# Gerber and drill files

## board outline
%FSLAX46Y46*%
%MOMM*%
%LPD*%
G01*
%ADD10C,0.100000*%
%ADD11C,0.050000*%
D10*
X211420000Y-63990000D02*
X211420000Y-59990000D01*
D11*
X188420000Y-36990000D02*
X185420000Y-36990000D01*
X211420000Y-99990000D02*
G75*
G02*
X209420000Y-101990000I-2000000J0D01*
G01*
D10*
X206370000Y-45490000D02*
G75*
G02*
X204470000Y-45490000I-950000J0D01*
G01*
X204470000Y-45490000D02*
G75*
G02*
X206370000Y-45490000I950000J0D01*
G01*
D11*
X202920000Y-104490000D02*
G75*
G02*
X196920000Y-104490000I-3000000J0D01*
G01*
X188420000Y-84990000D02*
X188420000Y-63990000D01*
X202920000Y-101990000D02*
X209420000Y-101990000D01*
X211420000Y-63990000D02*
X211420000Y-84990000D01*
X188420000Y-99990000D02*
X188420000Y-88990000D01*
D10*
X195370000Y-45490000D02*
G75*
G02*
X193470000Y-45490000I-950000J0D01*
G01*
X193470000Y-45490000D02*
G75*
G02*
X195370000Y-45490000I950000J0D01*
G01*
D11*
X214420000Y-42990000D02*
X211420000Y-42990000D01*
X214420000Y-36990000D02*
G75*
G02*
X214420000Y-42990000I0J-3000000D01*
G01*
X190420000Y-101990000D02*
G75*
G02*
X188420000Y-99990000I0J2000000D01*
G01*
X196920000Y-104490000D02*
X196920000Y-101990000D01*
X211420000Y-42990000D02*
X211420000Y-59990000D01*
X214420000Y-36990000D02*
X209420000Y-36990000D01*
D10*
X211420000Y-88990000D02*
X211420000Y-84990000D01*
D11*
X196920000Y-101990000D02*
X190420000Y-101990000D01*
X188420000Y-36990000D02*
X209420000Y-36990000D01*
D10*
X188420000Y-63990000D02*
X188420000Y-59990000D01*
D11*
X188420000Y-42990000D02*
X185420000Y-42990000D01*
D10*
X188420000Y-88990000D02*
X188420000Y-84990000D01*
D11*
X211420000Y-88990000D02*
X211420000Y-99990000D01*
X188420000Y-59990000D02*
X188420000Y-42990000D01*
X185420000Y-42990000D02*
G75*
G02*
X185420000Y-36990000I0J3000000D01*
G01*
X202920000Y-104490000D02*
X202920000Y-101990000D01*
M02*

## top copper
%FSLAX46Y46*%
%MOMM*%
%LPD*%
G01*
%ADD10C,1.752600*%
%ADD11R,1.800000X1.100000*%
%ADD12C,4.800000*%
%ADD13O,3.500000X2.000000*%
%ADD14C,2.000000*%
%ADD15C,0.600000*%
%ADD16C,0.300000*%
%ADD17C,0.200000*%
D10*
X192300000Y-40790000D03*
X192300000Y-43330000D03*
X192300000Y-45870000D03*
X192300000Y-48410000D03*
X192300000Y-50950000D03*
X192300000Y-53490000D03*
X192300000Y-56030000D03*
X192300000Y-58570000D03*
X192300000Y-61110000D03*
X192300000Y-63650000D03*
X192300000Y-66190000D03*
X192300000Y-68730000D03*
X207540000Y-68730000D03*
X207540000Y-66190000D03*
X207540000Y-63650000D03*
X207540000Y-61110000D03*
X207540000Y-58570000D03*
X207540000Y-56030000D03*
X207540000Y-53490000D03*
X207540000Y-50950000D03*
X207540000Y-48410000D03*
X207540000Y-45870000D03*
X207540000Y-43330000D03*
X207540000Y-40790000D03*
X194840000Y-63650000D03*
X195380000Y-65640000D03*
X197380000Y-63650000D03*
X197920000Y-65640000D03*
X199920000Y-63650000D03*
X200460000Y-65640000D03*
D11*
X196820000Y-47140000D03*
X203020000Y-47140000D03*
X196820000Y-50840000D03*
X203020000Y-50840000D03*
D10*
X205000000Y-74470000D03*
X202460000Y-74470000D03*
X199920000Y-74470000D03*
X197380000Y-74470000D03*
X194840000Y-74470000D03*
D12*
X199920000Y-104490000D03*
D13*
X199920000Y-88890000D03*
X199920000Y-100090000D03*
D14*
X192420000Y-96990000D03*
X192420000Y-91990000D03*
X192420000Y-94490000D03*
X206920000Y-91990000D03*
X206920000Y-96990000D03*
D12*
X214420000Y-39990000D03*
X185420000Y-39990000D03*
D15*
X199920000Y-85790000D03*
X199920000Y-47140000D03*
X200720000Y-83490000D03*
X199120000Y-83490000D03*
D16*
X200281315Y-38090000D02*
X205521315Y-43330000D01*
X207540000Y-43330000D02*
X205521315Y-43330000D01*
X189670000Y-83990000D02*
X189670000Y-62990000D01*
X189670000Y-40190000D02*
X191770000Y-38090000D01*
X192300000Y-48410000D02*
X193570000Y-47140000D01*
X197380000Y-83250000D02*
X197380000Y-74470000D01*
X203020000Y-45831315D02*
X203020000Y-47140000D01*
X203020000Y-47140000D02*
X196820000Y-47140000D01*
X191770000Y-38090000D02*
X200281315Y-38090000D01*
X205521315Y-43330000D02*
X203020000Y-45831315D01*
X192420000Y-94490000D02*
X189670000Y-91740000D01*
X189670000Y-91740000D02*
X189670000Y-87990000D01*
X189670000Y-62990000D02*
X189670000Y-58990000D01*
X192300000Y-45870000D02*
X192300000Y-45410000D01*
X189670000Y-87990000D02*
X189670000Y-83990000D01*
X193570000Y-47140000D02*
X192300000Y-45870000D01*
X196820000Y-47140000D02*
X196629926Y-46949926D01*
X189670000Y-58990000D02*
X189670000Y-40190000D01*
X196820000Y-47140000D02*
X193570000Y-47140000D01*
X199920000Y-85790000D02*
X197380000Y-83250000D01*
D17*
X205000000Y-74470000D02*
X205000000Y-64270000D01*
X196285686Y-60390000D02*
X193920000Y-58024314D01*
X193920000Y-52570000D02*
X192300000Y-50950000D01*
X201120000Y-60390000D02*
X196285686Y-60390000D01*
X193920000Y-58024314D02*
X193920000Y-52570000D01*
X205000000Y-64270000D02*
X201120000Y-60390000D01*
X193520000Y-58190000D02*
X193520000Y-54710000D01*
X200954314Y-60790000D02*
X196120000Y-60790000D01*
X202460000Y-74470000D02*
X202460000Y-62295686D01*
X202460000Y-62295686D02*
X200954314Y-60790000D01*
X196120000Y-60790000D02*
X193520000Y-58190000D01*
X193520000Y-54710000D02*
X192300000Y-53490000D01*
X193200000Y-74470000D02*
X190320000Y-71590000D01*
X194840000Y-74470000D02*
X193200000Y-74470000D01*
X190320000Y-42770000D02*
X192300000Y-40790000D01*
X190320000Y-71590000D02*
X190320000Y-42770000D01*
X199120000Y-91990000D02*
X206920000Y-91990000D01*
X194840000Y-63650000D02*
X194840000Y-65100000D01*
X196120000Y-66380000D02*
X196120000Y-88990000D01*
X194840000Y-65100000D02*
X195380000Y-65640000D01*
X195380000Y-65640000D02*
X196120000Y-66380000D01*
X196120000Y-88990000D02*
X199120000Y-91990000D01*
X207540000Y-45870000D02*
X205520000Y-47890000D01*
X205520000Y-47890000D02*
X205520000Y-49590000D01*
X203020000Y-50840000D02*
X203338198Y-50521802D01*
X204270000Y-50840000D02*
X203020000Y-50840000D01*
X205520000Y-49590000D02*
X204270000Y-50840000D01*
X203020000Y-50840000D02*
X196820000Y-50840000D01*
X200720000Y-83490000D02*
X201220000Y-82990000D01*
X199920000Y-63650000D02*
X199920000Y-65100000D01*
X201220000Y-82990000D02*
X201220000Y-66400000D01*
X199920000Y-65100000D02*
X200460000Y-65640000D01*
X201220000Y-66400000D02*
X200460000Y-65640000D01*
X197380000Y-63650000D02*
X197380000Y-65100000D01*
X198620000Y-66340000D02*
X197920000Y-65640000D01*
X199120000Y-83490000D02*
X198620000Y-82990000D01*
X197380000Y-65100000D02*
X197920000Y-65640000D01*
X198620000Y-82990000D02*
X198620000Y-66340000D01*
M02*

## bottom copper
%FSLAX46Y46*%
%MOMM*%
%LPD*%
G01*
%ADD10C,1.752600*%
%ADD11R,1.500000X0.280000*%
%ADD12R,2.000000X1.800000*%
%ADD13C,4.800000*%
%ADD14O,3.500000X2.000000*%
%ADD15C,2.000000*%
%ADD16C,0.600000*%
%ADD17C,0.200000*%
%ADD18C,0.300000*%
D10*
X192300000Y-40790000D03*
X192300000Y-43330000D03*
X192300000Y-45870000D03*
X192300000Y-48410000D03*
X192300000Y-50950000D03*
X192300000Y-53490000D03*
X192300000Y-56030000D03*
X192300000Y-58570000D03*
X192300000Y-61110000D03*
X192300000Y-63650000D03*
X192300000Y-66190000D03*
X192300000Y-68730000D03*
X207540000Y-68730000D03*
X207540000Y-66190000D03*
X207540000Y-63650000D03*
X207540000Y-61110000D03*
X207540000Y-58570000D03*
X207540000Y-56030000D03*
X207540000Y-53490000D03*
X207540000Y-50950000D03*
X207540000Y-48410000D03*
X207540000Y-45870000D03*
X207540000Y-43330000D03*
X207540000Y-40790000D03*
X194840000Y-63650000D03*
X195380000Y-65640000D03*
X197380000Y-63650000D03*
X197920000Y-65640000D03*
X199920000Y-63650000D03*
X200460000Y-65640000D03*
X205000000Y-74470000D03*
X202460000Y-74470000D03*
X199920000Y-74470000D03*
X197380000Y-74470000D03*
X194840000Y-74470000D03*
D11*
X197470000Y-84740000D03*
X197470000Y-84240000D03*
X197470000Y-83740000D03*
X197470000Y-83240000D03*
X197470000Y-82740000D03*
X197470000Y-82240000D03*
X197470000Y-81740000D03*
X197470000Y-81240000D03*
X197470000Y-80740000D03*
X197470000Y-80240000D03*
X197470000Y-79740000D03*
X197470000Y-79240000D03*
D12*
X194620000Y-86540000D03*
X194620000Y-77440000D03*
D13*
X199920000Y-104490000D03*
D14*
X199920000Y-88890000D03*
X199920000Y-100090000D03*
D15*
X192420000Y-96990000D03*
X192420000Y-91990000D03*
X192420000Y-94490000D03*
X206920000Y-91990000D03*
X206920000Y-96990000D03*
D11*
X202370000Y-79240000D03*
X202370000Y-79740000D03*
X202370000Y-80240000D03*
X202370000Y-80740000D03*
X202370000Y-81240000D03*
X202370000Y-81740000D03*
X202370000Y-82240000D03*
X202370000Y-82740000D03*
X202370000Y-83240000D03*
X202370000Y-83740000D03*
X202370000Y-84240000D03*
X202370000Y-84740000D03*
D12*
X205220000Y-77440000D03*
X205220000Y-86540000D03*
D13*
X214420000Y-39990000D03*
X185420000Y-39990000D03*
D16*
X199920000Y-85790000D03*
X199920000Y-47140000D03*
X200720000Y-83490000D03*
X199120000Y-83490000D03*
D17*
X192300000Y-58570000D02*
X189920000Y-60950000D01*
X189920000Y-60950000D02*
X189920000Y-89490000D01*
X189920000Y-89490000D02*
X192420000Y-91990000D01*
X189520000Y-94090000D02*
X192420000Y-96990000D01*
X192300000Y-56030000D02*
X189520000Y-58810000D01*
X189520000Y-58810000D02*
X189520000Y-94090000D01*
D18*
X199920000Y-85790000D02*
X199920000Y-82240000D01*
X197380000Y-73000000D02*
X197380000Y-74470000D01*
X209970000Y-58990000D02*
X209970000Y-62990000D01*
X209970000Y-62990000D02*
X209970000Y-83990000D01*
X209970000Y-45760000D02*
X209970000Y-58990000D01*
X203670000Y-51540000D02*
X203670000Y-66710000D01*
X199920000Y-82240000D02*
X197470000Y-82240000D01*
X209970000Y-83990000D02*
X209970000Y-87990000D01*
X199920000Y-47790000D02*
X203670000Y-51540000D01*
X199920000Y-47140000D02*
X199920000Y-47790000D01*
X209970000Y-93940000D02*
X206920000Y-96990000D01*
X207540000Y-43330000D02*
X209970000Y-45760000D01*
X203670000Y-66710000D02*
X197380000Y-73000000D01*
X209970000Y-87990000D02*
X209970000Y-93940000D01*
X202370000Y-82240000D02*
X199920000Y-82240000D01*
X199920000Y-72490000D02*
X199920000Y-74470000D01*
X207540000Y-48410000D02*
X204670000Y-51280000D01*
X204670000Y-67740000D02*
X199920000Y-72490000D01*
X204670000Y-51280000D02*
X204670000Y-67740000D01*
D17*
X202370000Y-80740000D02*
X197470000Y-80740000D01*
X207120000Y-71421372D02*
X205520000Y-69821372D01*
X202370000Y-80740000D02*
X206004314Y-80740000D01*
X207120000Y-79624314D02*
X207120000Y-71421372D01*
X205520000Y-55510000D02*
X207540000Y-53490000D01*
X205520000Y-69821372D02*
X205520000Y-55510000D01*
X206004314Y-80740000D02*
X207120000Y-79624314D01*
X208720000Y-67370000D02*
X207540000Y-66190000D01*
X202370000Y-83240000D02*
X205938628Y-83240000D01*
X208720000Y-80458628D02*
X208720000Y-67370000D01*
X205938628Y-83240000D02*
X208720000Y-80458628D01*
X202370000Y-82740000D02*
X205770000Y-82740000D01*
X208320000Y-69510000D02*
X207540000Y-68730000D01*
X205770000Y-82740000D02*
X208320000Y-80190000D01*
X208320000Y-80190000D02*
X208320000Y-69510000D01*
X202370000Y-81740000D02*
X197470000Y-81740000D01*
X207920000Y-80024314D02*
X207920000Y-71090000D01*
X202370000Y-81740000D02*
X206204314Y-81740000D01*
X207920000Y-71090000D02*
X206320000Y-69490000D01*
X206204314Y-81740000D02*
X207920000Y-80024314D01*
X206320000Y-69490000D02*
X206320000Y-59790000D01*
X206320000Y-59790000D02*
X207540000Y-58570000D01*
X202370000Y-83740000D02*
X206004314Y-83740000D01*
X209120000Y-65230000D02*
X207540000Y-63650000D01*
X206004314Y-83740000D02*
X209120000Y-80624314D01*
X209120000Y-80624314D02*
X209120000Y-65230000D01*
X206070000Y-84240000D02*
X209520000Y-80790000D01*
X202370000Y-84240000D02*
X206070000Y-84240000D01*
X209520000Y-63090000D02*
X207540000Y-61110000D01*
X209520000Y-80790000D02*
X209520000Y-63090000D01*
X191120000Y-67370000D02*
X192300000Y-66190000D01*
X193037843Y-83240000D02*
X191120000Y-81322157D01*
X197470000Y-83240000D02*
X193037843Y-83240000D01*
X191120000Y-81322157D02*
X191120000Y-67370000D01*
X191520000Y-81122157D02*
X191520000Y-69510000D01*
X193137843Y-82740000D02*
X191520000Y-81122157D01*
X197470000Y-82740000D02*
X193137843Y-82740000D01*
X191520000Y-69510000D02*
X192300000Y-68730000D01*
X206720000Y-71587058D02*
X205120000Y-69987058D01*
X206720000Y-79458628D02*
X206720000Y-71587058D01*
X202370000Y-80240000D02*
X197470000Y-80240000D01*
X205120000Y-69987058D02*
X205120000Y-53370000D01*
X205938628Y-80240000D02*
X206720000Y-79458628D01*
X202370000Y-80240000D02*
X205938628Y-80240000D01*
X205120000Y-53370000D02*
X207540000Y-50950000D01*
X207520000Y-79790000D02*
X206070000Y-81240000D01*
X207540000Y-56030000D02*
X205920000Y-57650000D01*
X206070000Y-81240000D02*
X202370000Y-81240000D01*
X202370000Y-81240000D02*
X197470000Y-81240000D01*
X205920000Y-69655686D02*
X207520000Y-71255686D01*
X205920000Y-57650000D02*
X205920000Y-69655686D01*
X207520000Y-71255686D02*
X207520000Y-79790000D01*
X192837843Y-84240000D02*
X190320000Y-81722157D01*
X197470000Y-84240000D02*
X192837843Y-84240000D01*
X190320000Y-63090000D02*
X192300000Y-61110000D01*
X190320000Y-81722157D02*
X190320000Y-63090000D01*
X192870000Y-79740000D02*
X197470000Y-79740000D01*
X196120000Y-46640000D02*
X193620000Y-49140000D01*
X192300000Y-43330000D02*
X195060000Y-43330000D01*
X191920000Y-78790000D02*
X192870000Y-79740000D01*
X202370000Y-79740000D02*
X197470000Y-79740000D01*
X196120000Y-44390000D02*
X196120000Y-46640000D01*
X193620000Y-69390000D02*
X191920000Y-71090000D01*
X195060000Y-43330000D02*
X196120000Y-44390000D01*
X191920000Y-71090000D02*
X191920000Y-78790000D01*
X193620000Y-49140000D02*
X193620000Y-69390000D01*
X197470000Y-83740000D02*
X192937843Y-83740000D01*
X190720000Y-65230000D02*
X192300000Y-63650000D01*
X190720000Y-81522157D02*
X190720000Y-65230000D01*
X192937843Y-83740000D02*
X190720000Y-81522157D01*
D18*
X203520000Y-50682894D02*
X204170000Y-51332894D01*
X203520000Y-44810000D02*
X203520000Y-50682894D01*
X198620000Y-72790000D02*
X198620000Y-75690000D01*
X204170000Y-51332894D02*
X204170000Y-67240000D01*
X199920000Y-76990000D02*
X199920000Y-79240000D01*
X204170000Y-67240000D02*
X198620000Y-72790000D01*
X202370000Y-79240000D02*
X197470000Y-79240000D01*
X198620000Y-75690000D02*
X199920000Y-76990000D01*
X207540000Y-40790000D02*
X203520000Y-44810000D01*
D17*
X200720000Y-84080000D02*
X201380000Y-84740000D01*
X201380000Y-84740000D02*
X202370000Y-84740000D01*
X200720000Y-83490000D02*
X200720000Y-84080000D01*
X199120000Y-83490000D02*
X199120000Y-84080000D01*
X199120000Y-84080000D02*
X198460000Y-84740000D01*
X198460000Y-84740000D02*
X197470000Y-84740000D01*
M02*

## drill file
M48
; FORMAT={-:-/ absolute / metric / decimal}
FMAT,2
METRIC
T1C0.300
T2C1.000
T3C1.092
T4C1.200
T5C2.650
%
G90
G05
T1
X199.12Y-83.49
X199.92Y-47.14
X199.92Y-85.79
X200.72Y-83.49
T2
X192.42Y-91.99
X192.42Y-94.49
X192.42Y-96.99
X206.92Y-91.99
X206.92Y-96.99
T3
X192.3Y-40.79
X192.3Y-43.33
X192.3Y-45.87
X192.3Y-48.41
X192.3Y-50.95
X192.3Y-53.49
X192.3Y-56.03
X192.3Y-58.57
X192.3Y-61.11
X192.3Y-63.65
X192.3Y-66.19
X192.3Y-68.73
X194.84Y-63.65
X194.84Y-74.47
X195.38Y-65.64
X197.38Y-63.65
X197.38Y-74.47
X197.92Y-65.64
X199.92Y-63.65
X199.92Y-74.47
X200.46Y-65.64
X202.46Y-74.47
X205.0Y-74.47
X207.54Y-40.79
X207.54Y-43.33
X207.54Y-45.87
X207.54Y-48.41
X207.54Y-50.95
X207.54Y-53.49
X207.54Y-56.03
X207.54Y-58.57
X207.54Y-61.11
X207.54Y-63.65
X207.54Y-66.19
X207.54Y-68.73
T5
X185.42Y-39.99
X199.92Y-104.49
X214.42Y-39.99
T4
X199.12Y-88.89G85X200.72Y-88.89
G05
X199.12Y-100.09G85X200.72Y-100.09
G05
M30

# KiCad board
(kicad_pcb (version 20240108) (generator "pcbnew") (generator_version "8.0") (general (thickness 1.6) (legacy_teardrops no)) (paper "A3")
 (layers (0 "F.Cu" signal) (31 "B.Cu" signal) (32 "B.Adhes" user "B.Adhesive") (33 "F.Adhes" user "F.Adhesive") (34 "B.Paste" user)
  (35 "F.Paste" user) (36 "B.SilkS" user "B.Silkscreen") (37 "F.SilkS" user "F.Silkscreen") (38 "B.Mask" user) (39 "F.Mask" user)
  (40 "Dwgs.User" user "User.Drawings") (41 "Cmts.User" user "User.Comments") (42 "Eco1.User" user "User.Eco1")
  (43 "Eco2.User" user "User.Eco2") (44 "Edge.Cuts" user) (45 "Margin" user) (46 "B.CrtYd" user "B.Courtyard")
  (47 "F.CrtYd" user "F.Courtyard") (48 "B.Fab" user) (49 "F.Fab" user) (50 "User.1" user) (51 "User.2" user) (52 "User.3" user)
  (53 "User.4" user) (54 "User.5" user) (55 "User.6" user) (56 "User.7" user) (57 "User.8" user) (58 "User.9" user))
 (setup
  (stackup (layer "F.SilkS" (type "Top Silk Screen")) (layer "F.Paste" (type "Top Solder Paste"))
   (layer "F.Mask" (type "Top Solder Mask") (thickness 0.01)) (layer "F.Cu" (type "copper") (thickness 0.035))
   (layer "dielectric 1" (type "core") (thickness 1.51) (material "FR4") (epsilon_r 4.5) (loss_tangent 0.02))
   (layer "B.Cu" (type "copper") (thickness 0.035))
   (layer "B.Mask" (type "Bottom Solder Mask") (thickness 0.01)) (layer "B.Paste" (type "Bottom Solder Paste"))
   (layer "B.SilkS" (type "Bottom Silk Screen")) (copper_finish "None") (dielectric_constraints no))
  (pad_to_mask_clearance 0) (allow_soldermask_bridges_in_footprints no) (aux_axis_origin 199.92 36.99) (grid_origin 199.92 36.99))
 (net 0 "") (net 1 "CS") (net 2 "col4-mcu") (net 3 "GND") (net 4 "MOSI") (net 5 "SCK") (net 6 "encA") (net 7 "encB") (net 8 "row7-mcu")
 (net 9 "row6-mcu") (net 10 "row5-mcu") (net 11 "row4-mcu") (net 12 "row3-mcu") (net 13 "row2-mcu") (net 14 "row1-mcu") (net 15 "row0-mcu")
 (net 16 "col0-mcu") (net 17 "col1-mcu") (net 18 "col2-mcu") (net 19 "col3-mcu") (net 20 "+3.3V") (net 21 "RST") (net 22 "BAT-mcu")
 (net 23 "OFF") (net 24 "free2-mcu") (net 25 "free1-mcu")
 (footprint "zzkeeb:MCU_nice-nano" (layer "F.Cu") (at 199.92 53.49)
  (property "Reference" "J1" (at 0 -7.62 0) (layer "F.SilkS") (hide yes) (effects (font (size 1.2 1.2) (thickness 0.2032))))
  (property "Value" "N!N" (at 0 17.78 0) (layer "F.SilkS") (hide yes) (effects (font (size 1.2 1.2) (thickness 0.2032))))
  (pad "1" thru_hole circle (at -7.62 -12.7 270) (size 1.7526 1.7526) (drill 1.0922) (layers "*.Cu" "*.Mask") (remove_unused_layers no)
   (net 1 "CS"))
  (pad "2" thru_hole circle (at -7.62 -10.16 270) (size 1.7526 1.7526) (drill 1.0922) (layers "*.Cu" "*.Mask") (remove_unused_layers no)
   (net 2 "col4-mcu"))
  (pad "3" thru_hole circle (at -7.62 -7.62 270) (size 1.7526 1.7526) (drill 1.0922) (layers "*.Cu" "*.Mask") (remove_unused_layers no)
   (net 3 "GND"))
  (pad "4" thru_hole circle (at -7.62 -5.08 270) (size 1.7526 1.7526) (drill 1.0922) (layers "*.Cu" "*.Mask") (remove_unused_layers no)
   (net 3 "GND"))
  (pad "5" thru_hole circle (at -7.62 -2.54 270) (size 1.7526 1.7526) (drill 1.0922) (layers "*.Cu" "*.Mask") (remove_unused_layers no)
   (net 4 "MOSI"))
  (pad "6" thru_hole circle (at -7.62 0 270) (size 1.7526 1.7526) (drill 1.0922) (layers "*.Cu" "*.Mask") (remove_unused_layers no)
   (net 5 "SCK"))
  (pad "7" thru_hole circle (at -7.62 2.54 270) (size 1.7526 1.7526) (drill 1.0922) (layers "*.Cu" "*.Mask") (remove_unused_layers no)
   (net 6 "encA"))
  (pad "8" thru_hole circle (at -7.62 5.08 270) (size 1.7526 1.7526) (drill 1.0922) (layers "*.Cu" "*.Mask") (remove_unused_layers no)
   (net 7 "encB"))
  (pad "9" thru_hole circle (at -7.62 7.62 270) (size 1.7526 1.7526) (drill 1.0922) (layers "*.Cu" "*.Mask") (remove_unused_layers no)
   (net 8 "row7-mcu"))
  (pad "10" thru_hole circle (at -7.62 10.16 270) (size 1.7526 1.7526) (drill 1.0922) (layers "*.Cu" "*.Mask") (remove_unused_layers no)
   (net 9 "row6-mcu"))
  (pad "11" thru_hole circle (at -7.62 12.7 270) (size 1.7526 1.7526) (drill 1.0922) (layers "*.Cu" "*.Mask") (remove_unused_layers no)
   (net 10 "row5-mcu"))
  (pad "12" thru_hole circle (at -7.62 15.24 270) (size 1.7526 1.7526) (drill 1.0922) (layers "*.Cu" "*.Mask") (remove_unused_layers no)
   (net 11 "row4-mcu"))
  (pad "13" thru_hole circle (at 7.62 15.24 270) (size 1.7526 1.7526) (drill 1.0922) (layers "*.Cu" "*.Mask") (remove_unused_layers no)
   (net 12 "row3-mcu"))
  (pad "14" thru_hole circle (at 7.62 12.7 270) (size 1.7526 1.7526) (drill 1.0922) (layers "*.Cu" "*.Mask") (remove_unused_layers no)
   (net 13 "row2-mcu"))
  (pad "15" thru_hole circle (at 7.62 10.16 270) (size 1.7526 1.7526) (drill 1.0922) (layers "*.Cu" "*.Mask") (remove_unused_layers no)
   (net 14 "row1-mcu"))
  (pad "16" thru_hole circle (at 7.62 7.62 270) (size 1.7526 1.7526) (drill 1.0922) (layers "*.Cu" "*.Mask") (remove_unused_layers no)
   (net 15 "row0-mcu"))
  (pad "17" thru_hole circle (at 7.62 5.08 270) (size 1.7526 1.7526) (drill 1.0922) (layers "*.Cu" "*.Mask") (remove_unused_layers no)
   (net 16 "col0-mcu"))
  (pad "18" thru_hole circle (at 7.62 2.54 270) (size 1.7526 1.7526) (drill 1.0922) (layers "*.Cu" "*.Mask") (remove_unused_layers no)
   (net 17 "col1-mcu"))
  (pad "19" thru_hole circle (at 7.62 0 270) (size 1.7526 1.7526) (drill 1.0922) (layers "*.Cu" "*.Mask") (remove_unused_layers no)
   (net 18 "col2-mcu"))
  (pad "20" thru_hole circle (at 7.62 -2.54 270) (size 1.7526 1.7526) (drill 1.0922) (layers "*.Cu" "*.Mask") (remove_unused_layers no)
   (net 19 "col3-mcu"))
  (pad "21" thru_hole circle (at 7.62 -5.08 270) (size 1.7526 1.7526) (drill 1.0922) (layers "*.Cu" "*.Mask") (remove_unused_layers no)
   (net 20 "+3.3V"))
  (pad "22" thru_hole circle (at 7.62 -7.62 270) (size 1.7526 1.7526) (drill 1.0922) (layers "*.Cu" "*.Mask") (remove_unused_layers no)
   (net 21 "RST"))
  (pad "23" thru_hole circle (at 7.62 -10.16 270) (size 1.7526 1.7526) (drill 1.0922) (layers "*.Cu" "*.Mask") (remove_unused_layers no)
   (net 3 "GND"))
  (pad "24" thru_hole circle (at 7.62 -12.7 270) (size 1.7526 1.7526) (drill 1.0922) (layers "*.Cu" "*.Mask") (remove_unused_layers no)
   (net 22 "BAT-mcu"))
  (pad "31" thru_hole circle (at -5.08 10.16 270) (size 1.7526 1.7526) (drill 1.0922) (layers "*.Cu" "*.Mask") (remove_unused_layers no)
   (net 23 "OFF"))
  (pad "31" thru_hole circle (at -4.54 12.15 270) (size 1.7526 1.7526) (drill 1.0922) (layers "*.Cu" "*.Mask") (remove_unused_layers no)
   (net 23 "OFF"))
  (pad "32" thru_hole circle (at -2.54 10.16 270) (size 1.7526 1.7526) (drill 1.0922) (layers "*.Cu" "*.Mask") (remove_unused_layers no)
   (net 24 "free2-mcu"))
  (pad "32" thru_hole circle (at -2 12.15 270) (size 1.7526 1.7526) (drill 1.0922) (layers "*.Cu" "*.Mask") (remove_unused_layers no)
   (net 24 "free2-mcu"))
  (pad "33" thru_hole circle (at 0 10.16 270) (size 1.7526 1.7526) (drill 1.0922) (layers "*.Cu" "*.Mask") (remove_unused_layers no)
   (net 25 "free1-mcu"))
  (pad "33" thru_hole circle (at 0.54 12.15 270) (size 1.7526 1.7526) (drill 1.0922) (layers "*.Cu" "*.Mask") (remove_unused_layers no)
   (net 25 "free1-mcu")))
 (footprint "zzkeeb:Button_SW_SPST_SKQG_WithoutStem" (layer "F.Cu") (at 199.92 48.99)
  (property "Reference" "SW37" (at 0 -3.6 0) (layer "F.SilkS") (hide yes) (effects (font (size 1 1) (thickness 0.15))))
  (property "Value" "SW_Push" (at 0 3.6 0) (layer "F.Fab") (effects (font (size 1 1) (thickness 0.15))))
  (pad "1" smd rect (at -3.1 -1.85) (size 1.8 1.1) (layers "F.Cu" "F.Paste" "F.Mask") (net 3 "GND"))
  (pad "1" smd rect (at 3.1 -1.85) (size 1.8 1.1) (layers "F.Cu" "F.Paste" "F.Mask") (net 3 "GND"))
  (pad "2" smd rect (at -3.1 1.85) (size 1.8 1.1) (layers "F.Cu" "F.Paste" "F.Mask") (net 21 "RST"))
  (pad "2" smd rect (at 3.1 1.85) (size 1.8 1.1) (layers "F.Cu" "F.Paste" "F.Mask") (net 21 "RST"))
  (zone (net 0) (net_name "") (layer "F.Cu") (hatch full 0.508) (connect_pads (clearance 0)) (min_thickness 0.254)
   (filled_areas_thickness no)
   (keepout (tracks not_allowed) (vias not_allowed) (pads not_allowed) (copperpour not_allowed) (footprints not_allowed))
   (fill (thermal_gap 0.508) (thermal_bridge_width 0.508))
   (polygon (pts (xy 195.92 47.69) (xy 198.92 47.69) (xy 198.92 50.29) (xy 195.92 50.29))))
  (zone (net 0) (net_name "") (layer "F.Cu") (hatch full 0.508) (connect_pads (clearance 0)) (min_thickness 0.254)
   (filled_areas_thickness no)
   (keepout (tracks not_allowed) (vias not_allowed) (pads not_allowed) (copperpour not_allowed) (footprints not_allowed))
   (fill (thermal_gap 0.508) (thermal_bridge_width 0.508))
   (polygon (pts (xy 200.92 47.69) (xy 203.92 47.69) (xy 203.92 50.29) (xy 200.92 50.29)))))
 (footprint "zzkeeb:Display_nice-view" (layer "B.Cu") (at 199.92 57.99 180)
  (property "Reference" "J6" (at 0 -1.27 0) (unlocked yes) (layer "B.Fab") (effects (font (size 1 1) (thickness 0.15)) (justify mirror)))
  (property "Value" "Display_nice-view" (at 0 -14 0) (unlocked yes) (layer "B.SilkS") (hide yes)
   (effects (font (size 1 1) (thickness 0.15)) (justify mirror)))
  (pad "1" thru_hole circle (at -5.08 -16.48 180) (size 1.7526 1.7526) (drill 1.0922) (layers "*.Cu" "*.Mask") (remove_unused_layers no)
   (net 4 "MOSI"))
  (pad "2" thru_hole circle (at -2.54 -16.48 180) (size 1.7526 1.7526) (drill 1.0922) (layers "*.Cu" "*.Mask") (remove_unused_layers no)
   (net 5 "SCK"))
  (pad "3" thru_hole circle (at 0 -16.48 180) (size 1.7526 1.7526) (drill 1.0922) (layers "*.Cu" "*.Mask") (remove_unused_layers no)
   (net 20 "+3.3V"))
  (pad "4" thru_hole circle (at 2.54 -16.48 180) (size 1.7526 1.7526) (drill 1.0922) (layers "*.Cu" "*.Mask") (remove_unused_layers no)
   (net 3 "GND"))
  (pad "5" thru_hole circle (at 5.08 -16.48 180) (size 1.7526 1.7526) (drill 1.0922) (layers "*.Cu" "*.Mask") (remove_unused_layers no)
   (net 1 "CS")))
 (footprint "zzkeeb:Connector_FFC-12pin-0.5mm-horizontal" (layer "B.Cu") (at 195.92 81.99 90)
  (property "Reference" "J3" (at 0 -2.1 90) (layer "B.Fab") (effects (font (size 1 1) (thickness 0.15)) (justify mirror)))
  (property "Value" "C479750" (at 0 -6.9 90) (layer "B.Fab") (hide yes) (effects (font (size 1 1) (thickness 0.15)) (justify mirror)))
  (pad "1" smd rect (at -2.75 1.55 90) (size 0.28 1.5) (layers "B.Cu" "B.Paste" "B.Mask") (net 24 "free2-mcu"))
  (pad "2" smd rect (at -2.25 1.55 90) (size 0.28 1.5) (layers "B.Cu" "B.Paste" "B.Mask") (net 8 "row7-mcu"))
  (pad "3" smd rect (at -1.75 1.55 90) (size 0.28 1.5) (layers "B.Cu" "B.Paste" "B.Mask") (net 9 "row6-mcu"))
  (pad "4" smd rect (at -1.25 1.55 90) (size 0.28 1.5) (layers "B.Cu" "B.Paste" "B.Mask") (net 10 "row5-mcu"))
  (pad "5" smd rect (at -0.75 1.55 90) (size 0.28 1.5) (layers "B.Cu" "B.Paste" "B.Mask") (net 11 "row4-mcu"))
  (pad "6" smd rect (at -0.25 1.55 90) (size 0.28 1.5) (layers "B.Cu" "B.Paste" "B.Mask") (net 3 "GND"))
  (pad "7" smd rect (at 0.25 1.55 90) (size 0.28 1.5) (layers "B.Cu" "B.Paste" "B.Mask") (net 16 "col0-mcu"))
  (pad "8" smd rect (at 0.75 1.55 90) (size 0.28 1.5) (layers "B.Cu" "B.Paste" "B.Mask") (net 17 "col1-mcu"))
  (pad "9" smd rect (at 1.25 1.55 90) (size 0.28 1.5) (layers "B.Cu" "B.Paste" "B.Mask") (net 18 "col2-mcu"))
  (pad "10" smd rect (at 1.75 1.55 90) (size 0.28 1.5) (layers "B.Cu" "B.Paste" "B.Mask") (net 19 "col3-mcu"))
  (pad "11" smd rect (at 2.25 1.55 90) (size 0.28 1.5) (layers "B.Cu" "B.Paste" "B.Mask") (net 2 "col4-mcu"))
  (pad "12" smd rect (at 2.75 1.55 90) (size 0.28 1.5) (layers "B.Cu" "B.Paste" "B.Mask") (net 22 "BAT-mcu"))
  (pad "MP" smd rect (at -4.55 -1.3 90) (size 1.8 2) (layers "B.Cu" "B.Paste" "B.Mask"))
  (pad "MP" smd rect (at 4.55 -1.3 90) (size 1.8 2) (layers "B.Cu" "B.Paste" "B.Mask")))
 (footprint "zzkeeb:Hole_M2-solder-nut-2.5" (layer "B.Cu") (at 199.92 104.49 180)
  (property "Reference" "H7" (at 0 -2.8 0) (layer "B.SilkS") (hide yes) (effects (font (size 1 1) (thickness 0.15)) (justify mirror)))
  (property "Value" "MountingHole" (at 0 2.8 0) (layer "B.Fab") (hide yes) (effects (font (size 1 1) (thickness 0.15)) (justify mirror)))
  (pad "" thru_hole circle (at 0 0 180) (size 4.8 4.8) (drill 2.65) (layers "*.Cu" "B.Mask") (remove_unused_layers no)))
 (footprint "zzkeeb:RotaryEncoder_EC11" (layer "B.Cu") (at 199.92 94.49)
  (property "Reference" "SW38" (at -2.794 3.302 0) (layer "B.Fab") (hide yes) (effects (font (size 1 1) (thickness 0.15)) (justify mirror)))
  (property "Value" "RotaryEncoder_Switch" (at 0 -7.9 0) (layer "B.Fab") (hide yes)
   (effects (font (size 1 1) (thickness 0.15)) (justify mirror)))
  (pad "" thru_hole oval (at 0 -5.6) (size 3.5 2) (drill oval 2.8 1.2) (layers "*.Cu" "*.Mask") (remove_unused_layers no))
  (pad "" thru_hole oval (at 0 5.6) (size 3.5 2) (drill oval 2.8 1.2) (layers "*.Cu" "*.Mask") (remove_unused_layers no))
  (pad "A" thru_hole circle (at -7.5 2.5) (size 2 2) (drill 1) (layers "*.Cu" "F.Mask") (remove_unused_layers no) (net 6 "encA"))
  (pad "B" thru_hole circle (at -7.5 -2.5) (size 2 2) (drill 1) (layers "*.Cu" "F.Mask") (remove_unused_layers no) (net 7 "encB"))
  (pad "C" thru_hole circle (at -7.5 0) (size 2 2) (drill 1) (layers "*.Cu" "F.Mask") (remove_unused_layers no) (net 3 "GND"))
  (pad "S1" thru_hole circle (at 7 -2.5) (size 2 2) (drill 1) (layers "*.Cu" "F.Mask") (remove_unused_layers no) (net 23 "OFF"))
  (pad "S2" thru_hole circle (at 7 2.5) (size 2 2) (drill 1) (layers "*.Cu" "F.Mask") (remove_unused_layers no) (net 3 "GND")))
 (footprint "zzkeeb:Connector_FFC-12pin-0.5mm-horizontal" (layer "B.Cu") (at 203.92 81.99 -90)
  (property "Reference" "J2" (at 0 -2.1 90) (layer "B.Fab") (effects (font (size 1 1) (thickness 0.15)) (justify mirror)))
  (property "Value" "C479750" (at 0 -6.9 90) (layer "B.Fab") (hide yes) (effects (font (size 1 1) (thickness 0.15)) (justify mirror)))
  (pad "1" smd rect (at -2.75 1.55 270) (size 0.28 1.5) (layers "B.Cu" "B.Paste" "B.Mask") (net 22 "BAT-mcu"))
  (pad "2" smd rect (at -2.25 1.55 270) (size 0.28 1.5) (layers "B.Cu" "B.Paste" "B.Mask") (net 2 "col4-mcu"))
  (pad "3" smd rect (at -1.75 1.55 270) (size 0.28 1.5) (layers "B.Cu" "B.Paste" "B.Mask") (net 19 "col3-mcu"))
  (pad "4" smd rect (at -1.25 1.55 270) (size 0.28 1.5) (layers "B.Cu" "B.Paste" "B.Mask") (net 18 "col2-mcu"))
  (pad "5" smd rect (at -0.75 1.55 270) (size 0.28 1.5) (layers "B.Cu" "B.Paste" "B.Mask") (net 17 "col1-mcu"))
  (pad "6" smd rect (at -0.25 1.55 270) (size 0.28 1.5) (layers "B.Cu" "B.Paste" "B.Mask") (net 16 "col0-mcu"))
  (pad "7" smd rect (at 0.25 1.55 270) (size 0.28 1.5) (layers "B.Cu" "B.Paste" "B.Mask") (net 3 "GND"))
  (pad "8" smd rect (at 0.75 1.55 270) (size 0.28 1.5) (layers "B.Cu" "B.Paste" "B.Mask") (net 12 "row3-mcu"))
  (pad "9" smd rect (at 1.25 1.55 270) (size 0.28 1.5) (layers "B.Cu" "B.Paste" "B.Mask") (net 13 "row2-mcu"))
  (pad "10" smd rect (at 1.75 1.55 270) (size 0.28 1.5) (layers "B.Cu" "B.Paste" "B.Mask") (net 14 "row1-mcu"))
  (pad "11" smd rect (at 2.25 1.55 270) (size 0.28 1.5) (layers "B.Cu" "B.Paste" "B.Mask") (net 15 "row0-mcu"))
  (pad "12" smd rect (at 2.75 1.55 270) (size 0.28 1.5) (layers "B.Cu" "B.Paste" "B.Mask") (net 25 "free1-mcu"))
  (pad "MP" smd rect (at -4.55 -1.3 270) (size 1.8 2) (layers "B.Cu" "B.Paste" "B.Mask"))
  (pad "MP" smd rect (at 4.55 -1.3 270) (size 1.8 2) (layers "B.Cu" "B.Paste" "B.Mask")))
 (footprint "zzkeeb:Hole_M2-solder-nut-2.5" (layer "B.Cu") (at 214.42 39.99 180)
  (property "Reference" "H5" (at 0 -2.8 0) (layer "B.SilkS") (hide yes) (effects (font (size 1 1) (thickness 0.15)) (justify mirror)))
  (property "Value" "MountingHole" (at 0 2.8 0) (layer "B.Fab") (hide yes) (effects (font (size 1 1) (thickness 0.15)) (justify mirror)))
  (pad "" thru_hole circle (at 0 0 180) (size 4.8 4.8) (drill 2.65) (layers "*.Cu" "B.Mask") (remove_unused_layers no)))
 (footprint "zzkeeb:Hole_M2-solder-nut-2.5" (layer "B.Cu") (at 185.42 39.99 180)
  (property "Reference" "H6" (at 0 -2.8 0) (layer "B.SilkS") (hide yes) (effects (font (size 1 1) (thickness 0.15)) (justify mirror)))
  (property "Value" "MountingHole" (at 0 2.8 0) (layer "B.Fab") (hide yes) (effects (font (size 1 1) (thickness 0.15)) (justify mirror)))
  (pad "" thru_hole circle (at 0 0 180) (size 4.8 4.8) (drill 2.65) (layers "*.Cu" "B.Mask") (remove_unused_layers no)))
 (gr_line (start 211.42 63.99) (end 211.42 59.99) (stroke (width 0.1) (type default)) (layer "Edge.Cuts"))
 (gr_line (start 188.42 36.99) (end 185.42 36.99) (stroke (width 0.05) (type default)) (layer "Edge.Cuts"))
 (gr_arc (start 211.42 99.99) (mid 210.834213 101.404212) (end 209.42 101.99) (stroke (width 0.05) (type default)) (layer "Edge.Cuts"))
 (gr_circle (center 205.42 45.49) (end 206.37 45.49) (stroke (width 0.1) (type default)) (fill none) (layer "Edge.Cuts"))
 (gr_arc (start 202.92 104.49) (mid 199.92 107.49) (end 196.92 104.49) (stroke (width 0.05) (type default)) (layer "Edge.Cuts"))
 (gr_line (start 188.42 84.99) (end 188.42 63.99) (stroke (width 0.05) (type default)) (layer "Edge.Cuts"))
 (gr_line (start 202.92 101.99) (end 209.42 101.99) (stroke (width 0.05) (type default)) (layer "Edge.Cuts"))
 (gr_line (start 211.42 63.99) (end 211.42 84.99) (stroke (width 0.05) (type default)) (layer "Edge.Cuts"))
 (gr_line (start 188.42 99.99) (end 188.42 88.99) (stroke (width 0.05) (type default)) (layer "Edge.Cuts"))
 (gr_circle (center 194.42 45.49) (end 195.37 45.49) (stroke (width 0.1) (type default)) (fill none) (layer "Edge.Cuts"))
 (gr_line (start 214.42 42.99) (end 211.42 42.99) (stroke (width 0.05) (type default)) (layer "Edge.Cuts"))
 (gr_arc (start 214.42 36.99) (mid 217.42 39.99) (end 214.42 42.99) (stroke (width 0.05) (type default)) (layer "Edge.Cuts"))
 (gr_arc (start 190.42 101.99) (mid 189.005786 101.404214) (end 188.42 99.99) (stroke (width 0.05) (type default)) (layer "Edge.Cuts"))
 (gr_line (start 196.92 104.49) (end 196.92 101.99) (stroke (width 0.05) (type default)) (layer "Edge.Cuts"))
 (gr_line (start 211.42 42.99) (end 211.42 59.99) (stroke (width 0.05) (type default)) (layer "Edge.Cuts"))
 (gr_line (start 214.42 36.99) (end 209.42 36.99) (stroke (width 0.05) (type default)) (layer "Edge.Cuts"))
 (gr_line (start 211.42 88.99) (end 211.42 84.99) (stroke (width 0.1) (type default)) (layer "Edge.Cuts"))
 (gr_line (start 196.92 101.99) (end 190.42 101.99) (stroke (width 0.05) (type default)) (layer "Edge.Cuts"))
 (gr_line (start 188.42 36.99) (end 209.42 36.99) (stroke (width 0.05) (type default)) (layer "Edge.Cuts"))
 (gr_line (start 188.42 63.99) (end 188.42 59.99) (stroke (width 0.1) (type default)) (layer "Edge.Cuts"))
 (gr_line (start 188.42 42.99) (end 185.42 42.99) (stroke (width 0.05) (type default)) (layer "Edge.Cuts"))
 (gr_line (start 188.42 88.99) (end 188.42 84.99) (stroke (width 0.1) (type default)) (layer "Edge.Cuts"))
 (gr_line (start 211.42 88.99) (end 211.42 99.99) (stroke (width 0.05) (type default)) (layer "Edge.Cuts"))
 (gr_line (start 188.42 59.99) (end 188.42 42.99) (stroke (width 0.05) (type default)) (layer "Edge.Cuts"))
 (gr_arc (start 185.42 42.99) (mid 182.42 39.99) (end 185.42 36.99) (stroke (width 0.05) (type default)) (layer "Edge.Cuts"))
 (gr_line (start 202.92 104.49) (end 202.92 101.99) (stroke (width 0.05) (type default)) (layer "Edge.Cuts"))
 (segment (start 192.3 58.57) (end 189.92 60.95) (width 0.2) (layer "B.Cu") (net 7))
 (segment (start 189.92 60.95) (end 189.92 89.49) (width 0.2) (layer "B.Cu") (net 7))
 (segment (start 189.92 89.49) (end 192.42 91.99) (width 0.2) (layer "B.Cu") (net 7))
 (segment (start 189.52 94.09) (end 192.42 96.99) (width 0.2) (layer "B.Cu") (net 6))
 (segment (start 192.3 56.03) (end 189.52 58.81) (width 0.2) (layer "B.Cu") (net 6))
 (segment (start 189.52 58.81) (end 189.52 94.09) (width 0.2) (layer "B.Cu") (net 6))
 (segment (start 200.281315 38.09) (end 205.521315 43.33) (width 0.3) (layer "F.Cu") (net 3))
 (segment (start 207.54 43.33) (end 205.521315 43.33) (width 0.3) (layer "F.Cu") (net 3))
 (segment (start 189.67 83.99) (end 189.67 62.99) (width 0.3) (layer "F.Cu") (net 3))
 (segment (start 189.67 40.19) (end 191.77 38.09) (width 0.3) (layer "F.Cu") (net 3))
 (segment (start 192.3 48.41) (end 193.57 47.14) (width 0.3) (layer "F.Cu") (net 3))
 (segment (start 197.38 83.25) (end 197.38 74.47) (width 0.3) (layer "F.Cu") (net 3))
 (segment (start 203.02 45.831315) (end 203.02 47.14) (width 0.3) (layer "F.Cu") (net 3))
 (segment (start 203.02 47.14) (end 196.82 47.14) (width 0.3) (layer "F.Cu") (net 3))
 (segment (start 191.77 38.09) (end 200.281315 38.09) (width 0.3) (layer "F.Cu") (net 3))
 (segment (start 205.521315 43.33) (end 203.02 45.831315) (width 0.3) (layer "F.Cu") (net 3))
 (segment (start 192.42 94.49) (end 189.67 91.74) (width 0.3) (layer "F.Cu") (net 3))
 (segment (start 189.67 91.74) (end 189.67 87.99) (width 0.3) (layer "F.Cu") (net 3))
 (segment (start 189.67 62.99) (end 189.67 58.99) (width 0.3) (layer "F.Cu") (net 3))
 (segment (start 192.3 45.87) (end 192.3 45.41) (width 0.3) (layer "F.Cu") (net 3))
 (segment (start 189.67 87.99) (end 189.67 83.99) (width 0.3) (layer "F.Cu") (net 3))
 (segment (start 193.57 47.14) (end 192.3 45.87) (width 0.3) (layer "F.Cu") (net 3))
 (segment (start 196.82 47.14) (end 196.629926 46.949926) (width 0.3) (layer "F.Cu") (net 3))
 (segment (start 189.67 58.99) (end 189.67 40.19) (width 0.3) (layer "F.Cu") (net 3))
 (segment (start 196.82 47.14) (end 193.57 47.14) (width 0.3) (layer "F.Cu") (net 3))
 (segment (start 199.92 85.79) (end 197.38 83.25) (width 0.3) (layer "F.Cu") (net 3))
 (via (at 199.92 85.79) (size 0.6) (drill 0.3) (layers "F.Cu" "B.Cu") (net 3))
 (via (at 199.92 47.14) (size 0.6) (drill 0.3) (layers "F.Cu" "B.Cu") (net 3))
 (segment (start 199.92 85.79) (end 199.92 82.24) (width 0.3) (layer "B.Cu") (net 3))
 (segment (start 197.38 73) (end 197.38 74.47) (width 0.3) (layer "B.Cu") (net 3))
 (segment (start 209.97 58.99) (end 209.97 62.99) (width 0.3) (layer "B.Cu") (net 3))
 (segment (start 209.97 62.99) (end 209.97 83.99) (width 0.3) (layer "B.Cu") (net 3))
 (segment (start 209.97 45.76) (end 209.97 58.99) (width 0.3) (layer "B.Cu") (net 3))
 (segment (start 203.67 51.54) (end 203.67 66.71) (width 0.3) (layer "B.Cu") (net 3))
 (segment (start 199.92 82.24) (end 197.47 82.24) (width 0.3) (layer "B.Cu") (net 3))
 (segment (start 209.97 83.99) (end 209.97 87.99) (width 0.3) (layer "B.Cu") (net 3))
 (segment (start 199.92 47.79) (end 203.67 51.54) (width 0.3) (layer "B.Cu") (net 3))
 (segment (start 199.92 47.14) (end 199.92 47.79) (width 0.3) (layer "B.Cu") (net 3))
 (segment (start 209.97 93.94) (end 206.92 96.99) (width 0.3) (layer "B.Cu") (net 3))
 (segment (start 207.54 43.33) (end 209.97 45.76) (width 0.3) (layer "B.Cu") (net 3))
 (segment (start 203.67 66.71) (end 197.38 73) (width 0.3) (layer "B.Cu") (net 3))
 (segment (start 209.97 87.99) (end 209.97 93.94) (width 0.3) (layer "B.Cu") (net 3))
 (segment (start 202.37 82.24) (end 199.92 82.24) (width 0.3) (layer "B.Cu") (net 3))
 (segment (start 205 74.47) (end 205 64.27) (width 0.2) (layer "F.Cu") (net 4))
 (segment (start 196.285686 60.39) (end 193.92 58.024314) (width 0.2) (layer "F.Cu") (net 4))
 (segment (start 193.92 52.57) (end 192.3 50.95) (width 0.2) (layer "F.Cu") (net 4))
 (segment (start 201.12 60.39) (end 196.285686 60.39) (width 0.2) (layer "F.Cu") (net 4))
 (segment (start 193.92 58.024314) (end 193.92 52.57) (width 0.2) (layer "F.Cu") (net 4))
 (segment (start 205 64.27) (end 201.12 60.39) (width 0.2) (layer "F.Cu") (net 4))
 (segment (start 193.52 58.19) (end 193.52 54.71) (width 0.2) (layer "F.Cu") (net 5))
 (segment (start 200.954314 60.79) (end 196.12 60.79) (width 0.2) (layer "F.Cu") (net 5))
 (segment (start 202.46 74.47) (end 202.46 62.295686) (width 0.2) (layer "F.Cu") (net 5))
 (segment (start 202.46 62.295686) (end 200.954314 60.79) (width 0.2) (layer "F.Cu") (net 5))
 (segment (start 196.12 60.79) (end 193.52 58.19) (width 0.2) (layer "F.Cu") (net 5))
 (segment (start 193.52 54.71) (end 192.3 53.49) (width 0.2) (layer "F.Cu") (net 5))
 (segment (start 199.92 72.49) (end 199.92 74.47) (width 0.3) (layer "B.Cu") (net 20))
 (segment (start 207.54 48.41) (end 204.67 51.28) (width 0.3) (layer "B.Cu") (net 20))
 (segment (start 204.67 67.74) (end 199.92 72.49) (width 0.3) (layer "B.Cu") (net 20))
 (segment (start 204.67 51.28) (end 204.67 67.74) (width 0.3) (layer "B.Cu") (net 20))
 (segment (start 193.2 74.47) (end 190.32 71.59) (width 0.2) (layer "F.Cu") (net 1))
 (segment (start 194.84 74.47) (end 193.2 74.47) (width 0.2) (layer "F.Cu") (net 1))
 (segment (start 190.32 42.77) (end 192.3 40.79) (width 0.2) (layer "F.Cu") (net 1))
 (segment (start 190.32 71.59) (end 190.32 42.77) (width 0.2) (layer "F.Cu") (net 1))
 (segment (start 199.12 91.99) (end 206.92 91.99) (width 0.2) (layer "F.Cu") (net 23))
 (segment (start 194.84 63.65) (end 194.84 65.1) (width 0.2) (layer "F.Cu") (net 23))
 (segment (start 196.12 66.38) (end 196.12 88.99) (width 0.2) (layer "F.Cu") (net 23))
 (segment (start 194.84 65.1) (end 195.38 65.64) (width 0.2) (layer "F.Cu") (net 23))
 (segment (start 195.38 65.64) (end 196.12 66.38) (width 0.2) (layer "F.Cu") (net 23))
 (segment (start 196.12 88.99) (end 199.12 91.99) (width 0.2) (layer "F.Cu") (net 23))
 (segment (start 207.54 45.87) (end 205.52 47.89) (width 0.2) (layer "F.Cu") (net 21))
 (segment (start 205.52 47.89) (end 205.52 49.59) (width 0.2) (layer "F.Cu") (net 21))
 (segment (start 203.02 50.84) (end 203.338198 50.521802) (width 0.2) (layer "F.Cu") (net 21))
 (segment (start 204.27 50.84) (end 203.02 50.84) (width 0.2) (layer "F.Cu") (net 21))
 (segment (start 205.52 49.59) (end 204.27 50.84) (width 0.2) (layer "F.Cu") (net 21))
 (segment (start 203.02 50.84) (end 196.82 50.84) (width 0.2) (layer "F.Cu") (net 21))
 (segment (start 202.37 80.74) (end 197.47 80.74) (width 0.2) (layer "B.Cu") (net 18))
 (segment (start 207.12 71.421372) (end 205.52 69.821372) (width 0.2) (layer "B.Cu") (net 18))
 (segment (start 202.37 80.74) (end 206.004314 80.74) (width 0.2) (layer "B.Cu") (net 18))
 (segment (start 207.12 79.624314) (end 207.12 71.421372) (width 0.2) (layer "B.Cu") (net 18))
 (segment (start 205.52 55.51) (end 207.54 53.49) (width 0.2) (layer "B.Cu") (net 18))
 (segment (start 205.52 69.821372) (end 205.52 55.51) (width 0.2) (layer "B.Cu") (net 18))
 (segment (start 206.004314 80.74) (end 207.12 79.624314) (width 0.2) (layer "B.Cu") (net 18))
 (segment (start 208.72 67.37) (end 207.54 66.19) (width 0.2) (layer "B.Cu") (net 13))
 (segment (start 202.37 83.24) (end 205.938628 83.24) (width 0.2) (layer "B.Cu") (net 13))
 (segment (start 208.72 80.458628) (end 208.72 67.37) (width 0.2) (layer "B.Cu") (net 13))
 (segment (start 205.938628 83.24) (end 208.72 80.458628) (width 0.2) (layer "B.Cu") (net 13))
 (segment (start 202.37 82.74) (end 205.77 82.74) (width 0.2) (layer "B.Cu") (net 12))
 (segment (start 208.32 69.51) (end 207.54 68.73) (width 0.2) (layer "B.Cu") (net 12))
 (segment (start 205.77 82.74) (end 208.32 80.19) (width 0.2) (layer "B.Cu") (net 12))
 (segment (start 208.32 80.19) (end 208.32 69.51) (width 0.2) (layer "B.Cu") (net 12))
 (segment (start 202.37 81.74) (end 197.47 81.74) (width 0.2) (layer "B.Cu") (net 16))
 (segment (start 207.92 80.024314) (end 207.92 71.09) (width 0.2) (layer "B.Cu") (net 16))
 (segment (start 202.37 81.74) (end 206.204314 81.74) (width 0.2) (layer "B.Cu") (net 16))
 (segment (start 207.92 71.09) (end 206.32 69.49) (width 0.2) (layer "B.Cu") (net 16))
 (segment (start 206.204314 81.74) (end 207.92 80.024314) (width 0.2) (layer "B.Cu") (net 16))
 (segment (start 206.32 69.49) (end 206.32 59.79) (width 0.2) (layer "B.Cu") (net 16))
 (segment (start 206.32 59.79) (end 207.54 58.57) (width 0.2) (layer "B.Cu") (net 16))
 (segment (start 202.37 83.74) (end 206.004314 83.74) (width 0.2) (layer "B.Cu") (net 14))
 (segment (start 209.12 65.23) (end 207.54 63.65) (width 0.2) (layer "B.Cu") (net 14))
 (segment (start 206.004314 83.74) (end 209.12 80.624314) (width 0.2) (layer "B.Cu") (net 14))
 (segment (start 209.12 80.624314) (end 209.12 65.23) (width 0.2) (layer "B.Cu") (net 14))
 (segment (start 206.07 84.24) (end 209.52 80.79) (width 0.2) (layer "B.Cu") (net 15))
 (segment (start 202.37 84.24) (end 206.07 84.24) (width 0.2) (layer "B.Cu") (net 15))
 (segment (start 209.52 63.09) (end 207.54 61.11) (width 0.2) (layer "B.Cu") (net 15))
 (segment (start 209.52 80.79) (end 209.52 63.09) (width 0.2) (layer "B.Cu") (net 15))
 (segment (start 191.12 67.37) (end 192.3 66.19) (width 0.2) (layer "B.Cu") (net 10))
 (segment (start 193.037843 83.24) (end 191.12 81.322157) (width 0.2) (layer "B.Cu") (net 10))
 (segment (start 197.47 83.24) (end 193.037843 83.24) (width 0.2) (layer "B.Cu") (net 10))
 (segment (start 191.12 81.322157) (end 191.12 67.37) (width 0.2) (layer "B.Cu") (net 10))
 (segment (start 191.52 81.122157) (end 191.52 69.51) (width 0.2) (layer "B.Cu") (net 11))
 (segment (start 193.137843 82.74) (end 191.52 81.122157) (width 0.2) (layer "B.Cu") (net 11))
 (segment (start 197.47 82.74) (end 193.137843 82.74) (width 0.2) (layer "B.Cu") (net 11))
 (segment (start 191.52 69.51) (end 192.3 68.73) (width 0.2) (layer "B.Cu") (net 11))
 (segment (start 206.72 71.587058) (end 205.12 69.987058) (width 0.2) (layer "B.Cu") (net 19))
 (segment (start 206.72 79.458628) (end 206.72 71.587058) (width 0.2) (layer "B.Cu") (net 19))
 (segment (start 202.37 80.24) (end 197.47 80.24) (width 0.2) (layer "B.Cu") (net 19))
 (segment (start 205.12 69.987058) (end 205.12 53.37) (width 0.2) (layer "B.Cu") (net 19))
 (segment (start 205.938628 80.24) (end 206.72 79.458628) (width 0.2) (layer "B.Cu") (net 19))
 (segment (start 202.37 80.24) (end 205.938628 80.24) (width 0.2) (layer "B.Cu") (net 19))
 (segment (start 205.12 53.37) (end 207.54 50.95) (width 0.2) (layer "B.Cu") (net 19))
 (segment (start 207.52 79.79) (end 206.07 81.24) (width 0.2) (layer "B.Cu") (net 17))
 (segment (start 207.54 56.03) (end 205.92 57.65) (width 0.2) (layer "B.Cu") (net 17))
 (segment (start 206.07 81.24) (end 202.37 81.24) (width 0.2) (layer "B.Cu") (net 17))
 (segment (start 202.37 81.24) (end 197.47 81.24) (width 0.2) (layer "B.Cu") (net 17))
 (segment (start 205.92 69.655686) (end 207.52 71.255686) (width 0.2) (layer "B.Cu") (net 17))
 (segment (start 205.92 57.65) (end 205.92 69.655686) (width 0.2) (layer "B.Cu") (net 17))
 (segment (start 207.52 71.255686) (end 207.52 79.79) (width 0.2) (layer "B.Cu") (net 17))
 (segment (start 192.837843 84.24) (end 190.32 81.722157) (width 0.2) (layer "B.Cu") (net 8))
 (segment (start 197.47 84.24) (end 192.837843 84.24) (width 0.2) (layer "B.Cu") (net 8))
 (segment (start 190.32 63.09) (end 192.3 61.11) (width 0.2) (layer "B.Cu") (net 8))
 (segment (start 190.32 81.722157) (end 190.32 63.09) (width 0.2) (layer "B.Cu") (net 8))
 (segment (start 192.87 79.74) (end 197.47 79.74) (width 0.2) (layer "B.Cu") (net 2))
 (segment (start 196.12 46.64) (end 193.62 49.14) (width 0.2) (layer "B.Cu") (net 2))
 (segment (start 192.3 43.33) (end 195.06 43.33) (width 0.2) (layer "B.Cu") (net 2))
 (segment (start 191.92 78.79) (end 192.87 79.74) (width 0.2) (layer "B.Cu") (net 2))
 (segment (start 202.37 79.74) (end 197.47 79.74) (width 0.2) (layer "B.Cu") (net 2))
 (segment (start 196.12 44.39) (end 196.12 46.64) (width 0.2) (layer "B.Cu") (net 2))
 (segment (start 193.62 69.39) (end 191.92 71.09) (width 0.2) (layer "B.Cu") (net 2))
 (segment (start 195.06 43.33) (end 196.12 44.39) (width 0.2) (layer "B.Cu") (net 2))
 (segment (start 191.92 71.09) (end 191.92 78.79) (width 0.2) (layer "B.Cu") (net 2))
 (segment (start 193.62 49.14) (end 193.62 69.39) (width 0.2) (layer "B.Cu") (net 2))
 (segment (start 197.47 83.74) (end 192.937843 83.74) (width 0.2) (layer "B.Cu") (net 9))
 (segment (start 190.72 65.23) (end 192.3 63.65) (width 0.2) (layer "B.Cu") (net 9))
 (segment (start 190.72 81.522157) (end 190.72 65.23) (width 0.2) (layer "B.Cu") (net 9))
 (segment (start 192.937843 83.74) (end 190.72 81.522157) (width 0.2) (layer "B.Cu") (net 9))
 (segment (start 203.52 50.682894) (end 204.17 51.332894) (width 0.3) (layer "B.Cu") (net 22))
 (segment (start 203.52 44.81) (end 203.52 50.682894) (width 0.3) (layer "B.Cu") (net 22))
 (segment (start 198.62 72.79) (end 198.62 75.69) (width 0.3) (layer "B.Cu") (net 22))
 (segment (start 204.17 51.332894) (end 204.17 67.24) (width 0.3) (layer "B.Cu") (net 22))
 (segment (start 199.92 76.99) (end 199.92 79.24) (width 0.3) (layer "B.Cu") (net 22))
 (segment (start 204.17 67.24) (end 198.62 72.79) (width 0.3) (layer "B.Cu") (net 22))
 (segment (start 202.37 79.24) (end 197.47 79.24) (width 0.3) (layer "B.Cu") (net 22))
 (segment (start 198.62 75.69) (end 199.92 76.99) (width 0.3) (layer "B.Cu") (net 22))
 (segment (start 207.54 40.79) (end 203.52 44.81) (width 0.3) (layer "B.Cu") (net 22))
 (segment (start 200.72 83.49) (end 201.22 82.99) (width 0.2) (layer "F.Cu") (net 25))
 (segment (start 199.92 63.65) (end 199.92 65.1) (width 0.2) (layer "F.Cu") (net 25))
 (segment (start 201.22 82.99) (end 201.22 66.4) (width 0.2) (layer "F.Cu") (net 25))
 (segment (start 199.92 65.1) (end 200.46 65.64) (width 0.2) (layer "F.Cu") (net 25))
 (segment (start 201.22 66.4) (end 200.46 65.64) (width 0.2) (layer "F.Cu") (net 25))
 (via (at 200.72 83.49) (size 0.6) (drill 0.3) (layers "F.Cu" "B.Cu") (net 25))
 (segment (start 200.72 84.08) (end 201.38 84.74) (width 0.2) (layer "B.Cu") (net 25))
 (segment (start 201.38 84.74) (end 202.37 84.74) (width 0.2) (layer "B.Cu") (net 25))
 (segment (start 200.72 83.49) (end 200.72 84.08) (width 0.2) (layer "B.Cu") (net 25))
 (segment (start 197.38 63.65) (end 197.38 65.1) (width 0.2) (layer "F.Cu") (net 24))
 (segment (start 198.62 66.34) (end 197.92 65.64) (width 0.2) (layer "F.Cu") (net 24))
 (segment (start 199.12 83.49) (end 198.62 82.99) (width 0.2) (layer "F.Cu") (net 24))
 (segment (start 197.38 65.1) (end 197.92 65.64) (width 0.2) (layer "F.Cu") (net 24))
 (segment (start 198.62 82.99) (end 198.62 66.34) (width 0.2) (layer "F.Cu") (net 24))
 (via (at 199.12 83.49) (size 0.6) (drill 0.3) (layers "F.Cu" "B.Cu") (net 24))
 (segment (start 199.12 83.49) (end 199.12 84.08) (width 0.2) (layer "B.Cu") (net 24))
 (segment (start 199.12 84.08) (end 198.46 84.74) (width 0.2) (layer "B.Cu") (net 24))
 (segment (start 198.46 84.74) (end 197.47 84.74) (width 0.2) (layer "B.Cu") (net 24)))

